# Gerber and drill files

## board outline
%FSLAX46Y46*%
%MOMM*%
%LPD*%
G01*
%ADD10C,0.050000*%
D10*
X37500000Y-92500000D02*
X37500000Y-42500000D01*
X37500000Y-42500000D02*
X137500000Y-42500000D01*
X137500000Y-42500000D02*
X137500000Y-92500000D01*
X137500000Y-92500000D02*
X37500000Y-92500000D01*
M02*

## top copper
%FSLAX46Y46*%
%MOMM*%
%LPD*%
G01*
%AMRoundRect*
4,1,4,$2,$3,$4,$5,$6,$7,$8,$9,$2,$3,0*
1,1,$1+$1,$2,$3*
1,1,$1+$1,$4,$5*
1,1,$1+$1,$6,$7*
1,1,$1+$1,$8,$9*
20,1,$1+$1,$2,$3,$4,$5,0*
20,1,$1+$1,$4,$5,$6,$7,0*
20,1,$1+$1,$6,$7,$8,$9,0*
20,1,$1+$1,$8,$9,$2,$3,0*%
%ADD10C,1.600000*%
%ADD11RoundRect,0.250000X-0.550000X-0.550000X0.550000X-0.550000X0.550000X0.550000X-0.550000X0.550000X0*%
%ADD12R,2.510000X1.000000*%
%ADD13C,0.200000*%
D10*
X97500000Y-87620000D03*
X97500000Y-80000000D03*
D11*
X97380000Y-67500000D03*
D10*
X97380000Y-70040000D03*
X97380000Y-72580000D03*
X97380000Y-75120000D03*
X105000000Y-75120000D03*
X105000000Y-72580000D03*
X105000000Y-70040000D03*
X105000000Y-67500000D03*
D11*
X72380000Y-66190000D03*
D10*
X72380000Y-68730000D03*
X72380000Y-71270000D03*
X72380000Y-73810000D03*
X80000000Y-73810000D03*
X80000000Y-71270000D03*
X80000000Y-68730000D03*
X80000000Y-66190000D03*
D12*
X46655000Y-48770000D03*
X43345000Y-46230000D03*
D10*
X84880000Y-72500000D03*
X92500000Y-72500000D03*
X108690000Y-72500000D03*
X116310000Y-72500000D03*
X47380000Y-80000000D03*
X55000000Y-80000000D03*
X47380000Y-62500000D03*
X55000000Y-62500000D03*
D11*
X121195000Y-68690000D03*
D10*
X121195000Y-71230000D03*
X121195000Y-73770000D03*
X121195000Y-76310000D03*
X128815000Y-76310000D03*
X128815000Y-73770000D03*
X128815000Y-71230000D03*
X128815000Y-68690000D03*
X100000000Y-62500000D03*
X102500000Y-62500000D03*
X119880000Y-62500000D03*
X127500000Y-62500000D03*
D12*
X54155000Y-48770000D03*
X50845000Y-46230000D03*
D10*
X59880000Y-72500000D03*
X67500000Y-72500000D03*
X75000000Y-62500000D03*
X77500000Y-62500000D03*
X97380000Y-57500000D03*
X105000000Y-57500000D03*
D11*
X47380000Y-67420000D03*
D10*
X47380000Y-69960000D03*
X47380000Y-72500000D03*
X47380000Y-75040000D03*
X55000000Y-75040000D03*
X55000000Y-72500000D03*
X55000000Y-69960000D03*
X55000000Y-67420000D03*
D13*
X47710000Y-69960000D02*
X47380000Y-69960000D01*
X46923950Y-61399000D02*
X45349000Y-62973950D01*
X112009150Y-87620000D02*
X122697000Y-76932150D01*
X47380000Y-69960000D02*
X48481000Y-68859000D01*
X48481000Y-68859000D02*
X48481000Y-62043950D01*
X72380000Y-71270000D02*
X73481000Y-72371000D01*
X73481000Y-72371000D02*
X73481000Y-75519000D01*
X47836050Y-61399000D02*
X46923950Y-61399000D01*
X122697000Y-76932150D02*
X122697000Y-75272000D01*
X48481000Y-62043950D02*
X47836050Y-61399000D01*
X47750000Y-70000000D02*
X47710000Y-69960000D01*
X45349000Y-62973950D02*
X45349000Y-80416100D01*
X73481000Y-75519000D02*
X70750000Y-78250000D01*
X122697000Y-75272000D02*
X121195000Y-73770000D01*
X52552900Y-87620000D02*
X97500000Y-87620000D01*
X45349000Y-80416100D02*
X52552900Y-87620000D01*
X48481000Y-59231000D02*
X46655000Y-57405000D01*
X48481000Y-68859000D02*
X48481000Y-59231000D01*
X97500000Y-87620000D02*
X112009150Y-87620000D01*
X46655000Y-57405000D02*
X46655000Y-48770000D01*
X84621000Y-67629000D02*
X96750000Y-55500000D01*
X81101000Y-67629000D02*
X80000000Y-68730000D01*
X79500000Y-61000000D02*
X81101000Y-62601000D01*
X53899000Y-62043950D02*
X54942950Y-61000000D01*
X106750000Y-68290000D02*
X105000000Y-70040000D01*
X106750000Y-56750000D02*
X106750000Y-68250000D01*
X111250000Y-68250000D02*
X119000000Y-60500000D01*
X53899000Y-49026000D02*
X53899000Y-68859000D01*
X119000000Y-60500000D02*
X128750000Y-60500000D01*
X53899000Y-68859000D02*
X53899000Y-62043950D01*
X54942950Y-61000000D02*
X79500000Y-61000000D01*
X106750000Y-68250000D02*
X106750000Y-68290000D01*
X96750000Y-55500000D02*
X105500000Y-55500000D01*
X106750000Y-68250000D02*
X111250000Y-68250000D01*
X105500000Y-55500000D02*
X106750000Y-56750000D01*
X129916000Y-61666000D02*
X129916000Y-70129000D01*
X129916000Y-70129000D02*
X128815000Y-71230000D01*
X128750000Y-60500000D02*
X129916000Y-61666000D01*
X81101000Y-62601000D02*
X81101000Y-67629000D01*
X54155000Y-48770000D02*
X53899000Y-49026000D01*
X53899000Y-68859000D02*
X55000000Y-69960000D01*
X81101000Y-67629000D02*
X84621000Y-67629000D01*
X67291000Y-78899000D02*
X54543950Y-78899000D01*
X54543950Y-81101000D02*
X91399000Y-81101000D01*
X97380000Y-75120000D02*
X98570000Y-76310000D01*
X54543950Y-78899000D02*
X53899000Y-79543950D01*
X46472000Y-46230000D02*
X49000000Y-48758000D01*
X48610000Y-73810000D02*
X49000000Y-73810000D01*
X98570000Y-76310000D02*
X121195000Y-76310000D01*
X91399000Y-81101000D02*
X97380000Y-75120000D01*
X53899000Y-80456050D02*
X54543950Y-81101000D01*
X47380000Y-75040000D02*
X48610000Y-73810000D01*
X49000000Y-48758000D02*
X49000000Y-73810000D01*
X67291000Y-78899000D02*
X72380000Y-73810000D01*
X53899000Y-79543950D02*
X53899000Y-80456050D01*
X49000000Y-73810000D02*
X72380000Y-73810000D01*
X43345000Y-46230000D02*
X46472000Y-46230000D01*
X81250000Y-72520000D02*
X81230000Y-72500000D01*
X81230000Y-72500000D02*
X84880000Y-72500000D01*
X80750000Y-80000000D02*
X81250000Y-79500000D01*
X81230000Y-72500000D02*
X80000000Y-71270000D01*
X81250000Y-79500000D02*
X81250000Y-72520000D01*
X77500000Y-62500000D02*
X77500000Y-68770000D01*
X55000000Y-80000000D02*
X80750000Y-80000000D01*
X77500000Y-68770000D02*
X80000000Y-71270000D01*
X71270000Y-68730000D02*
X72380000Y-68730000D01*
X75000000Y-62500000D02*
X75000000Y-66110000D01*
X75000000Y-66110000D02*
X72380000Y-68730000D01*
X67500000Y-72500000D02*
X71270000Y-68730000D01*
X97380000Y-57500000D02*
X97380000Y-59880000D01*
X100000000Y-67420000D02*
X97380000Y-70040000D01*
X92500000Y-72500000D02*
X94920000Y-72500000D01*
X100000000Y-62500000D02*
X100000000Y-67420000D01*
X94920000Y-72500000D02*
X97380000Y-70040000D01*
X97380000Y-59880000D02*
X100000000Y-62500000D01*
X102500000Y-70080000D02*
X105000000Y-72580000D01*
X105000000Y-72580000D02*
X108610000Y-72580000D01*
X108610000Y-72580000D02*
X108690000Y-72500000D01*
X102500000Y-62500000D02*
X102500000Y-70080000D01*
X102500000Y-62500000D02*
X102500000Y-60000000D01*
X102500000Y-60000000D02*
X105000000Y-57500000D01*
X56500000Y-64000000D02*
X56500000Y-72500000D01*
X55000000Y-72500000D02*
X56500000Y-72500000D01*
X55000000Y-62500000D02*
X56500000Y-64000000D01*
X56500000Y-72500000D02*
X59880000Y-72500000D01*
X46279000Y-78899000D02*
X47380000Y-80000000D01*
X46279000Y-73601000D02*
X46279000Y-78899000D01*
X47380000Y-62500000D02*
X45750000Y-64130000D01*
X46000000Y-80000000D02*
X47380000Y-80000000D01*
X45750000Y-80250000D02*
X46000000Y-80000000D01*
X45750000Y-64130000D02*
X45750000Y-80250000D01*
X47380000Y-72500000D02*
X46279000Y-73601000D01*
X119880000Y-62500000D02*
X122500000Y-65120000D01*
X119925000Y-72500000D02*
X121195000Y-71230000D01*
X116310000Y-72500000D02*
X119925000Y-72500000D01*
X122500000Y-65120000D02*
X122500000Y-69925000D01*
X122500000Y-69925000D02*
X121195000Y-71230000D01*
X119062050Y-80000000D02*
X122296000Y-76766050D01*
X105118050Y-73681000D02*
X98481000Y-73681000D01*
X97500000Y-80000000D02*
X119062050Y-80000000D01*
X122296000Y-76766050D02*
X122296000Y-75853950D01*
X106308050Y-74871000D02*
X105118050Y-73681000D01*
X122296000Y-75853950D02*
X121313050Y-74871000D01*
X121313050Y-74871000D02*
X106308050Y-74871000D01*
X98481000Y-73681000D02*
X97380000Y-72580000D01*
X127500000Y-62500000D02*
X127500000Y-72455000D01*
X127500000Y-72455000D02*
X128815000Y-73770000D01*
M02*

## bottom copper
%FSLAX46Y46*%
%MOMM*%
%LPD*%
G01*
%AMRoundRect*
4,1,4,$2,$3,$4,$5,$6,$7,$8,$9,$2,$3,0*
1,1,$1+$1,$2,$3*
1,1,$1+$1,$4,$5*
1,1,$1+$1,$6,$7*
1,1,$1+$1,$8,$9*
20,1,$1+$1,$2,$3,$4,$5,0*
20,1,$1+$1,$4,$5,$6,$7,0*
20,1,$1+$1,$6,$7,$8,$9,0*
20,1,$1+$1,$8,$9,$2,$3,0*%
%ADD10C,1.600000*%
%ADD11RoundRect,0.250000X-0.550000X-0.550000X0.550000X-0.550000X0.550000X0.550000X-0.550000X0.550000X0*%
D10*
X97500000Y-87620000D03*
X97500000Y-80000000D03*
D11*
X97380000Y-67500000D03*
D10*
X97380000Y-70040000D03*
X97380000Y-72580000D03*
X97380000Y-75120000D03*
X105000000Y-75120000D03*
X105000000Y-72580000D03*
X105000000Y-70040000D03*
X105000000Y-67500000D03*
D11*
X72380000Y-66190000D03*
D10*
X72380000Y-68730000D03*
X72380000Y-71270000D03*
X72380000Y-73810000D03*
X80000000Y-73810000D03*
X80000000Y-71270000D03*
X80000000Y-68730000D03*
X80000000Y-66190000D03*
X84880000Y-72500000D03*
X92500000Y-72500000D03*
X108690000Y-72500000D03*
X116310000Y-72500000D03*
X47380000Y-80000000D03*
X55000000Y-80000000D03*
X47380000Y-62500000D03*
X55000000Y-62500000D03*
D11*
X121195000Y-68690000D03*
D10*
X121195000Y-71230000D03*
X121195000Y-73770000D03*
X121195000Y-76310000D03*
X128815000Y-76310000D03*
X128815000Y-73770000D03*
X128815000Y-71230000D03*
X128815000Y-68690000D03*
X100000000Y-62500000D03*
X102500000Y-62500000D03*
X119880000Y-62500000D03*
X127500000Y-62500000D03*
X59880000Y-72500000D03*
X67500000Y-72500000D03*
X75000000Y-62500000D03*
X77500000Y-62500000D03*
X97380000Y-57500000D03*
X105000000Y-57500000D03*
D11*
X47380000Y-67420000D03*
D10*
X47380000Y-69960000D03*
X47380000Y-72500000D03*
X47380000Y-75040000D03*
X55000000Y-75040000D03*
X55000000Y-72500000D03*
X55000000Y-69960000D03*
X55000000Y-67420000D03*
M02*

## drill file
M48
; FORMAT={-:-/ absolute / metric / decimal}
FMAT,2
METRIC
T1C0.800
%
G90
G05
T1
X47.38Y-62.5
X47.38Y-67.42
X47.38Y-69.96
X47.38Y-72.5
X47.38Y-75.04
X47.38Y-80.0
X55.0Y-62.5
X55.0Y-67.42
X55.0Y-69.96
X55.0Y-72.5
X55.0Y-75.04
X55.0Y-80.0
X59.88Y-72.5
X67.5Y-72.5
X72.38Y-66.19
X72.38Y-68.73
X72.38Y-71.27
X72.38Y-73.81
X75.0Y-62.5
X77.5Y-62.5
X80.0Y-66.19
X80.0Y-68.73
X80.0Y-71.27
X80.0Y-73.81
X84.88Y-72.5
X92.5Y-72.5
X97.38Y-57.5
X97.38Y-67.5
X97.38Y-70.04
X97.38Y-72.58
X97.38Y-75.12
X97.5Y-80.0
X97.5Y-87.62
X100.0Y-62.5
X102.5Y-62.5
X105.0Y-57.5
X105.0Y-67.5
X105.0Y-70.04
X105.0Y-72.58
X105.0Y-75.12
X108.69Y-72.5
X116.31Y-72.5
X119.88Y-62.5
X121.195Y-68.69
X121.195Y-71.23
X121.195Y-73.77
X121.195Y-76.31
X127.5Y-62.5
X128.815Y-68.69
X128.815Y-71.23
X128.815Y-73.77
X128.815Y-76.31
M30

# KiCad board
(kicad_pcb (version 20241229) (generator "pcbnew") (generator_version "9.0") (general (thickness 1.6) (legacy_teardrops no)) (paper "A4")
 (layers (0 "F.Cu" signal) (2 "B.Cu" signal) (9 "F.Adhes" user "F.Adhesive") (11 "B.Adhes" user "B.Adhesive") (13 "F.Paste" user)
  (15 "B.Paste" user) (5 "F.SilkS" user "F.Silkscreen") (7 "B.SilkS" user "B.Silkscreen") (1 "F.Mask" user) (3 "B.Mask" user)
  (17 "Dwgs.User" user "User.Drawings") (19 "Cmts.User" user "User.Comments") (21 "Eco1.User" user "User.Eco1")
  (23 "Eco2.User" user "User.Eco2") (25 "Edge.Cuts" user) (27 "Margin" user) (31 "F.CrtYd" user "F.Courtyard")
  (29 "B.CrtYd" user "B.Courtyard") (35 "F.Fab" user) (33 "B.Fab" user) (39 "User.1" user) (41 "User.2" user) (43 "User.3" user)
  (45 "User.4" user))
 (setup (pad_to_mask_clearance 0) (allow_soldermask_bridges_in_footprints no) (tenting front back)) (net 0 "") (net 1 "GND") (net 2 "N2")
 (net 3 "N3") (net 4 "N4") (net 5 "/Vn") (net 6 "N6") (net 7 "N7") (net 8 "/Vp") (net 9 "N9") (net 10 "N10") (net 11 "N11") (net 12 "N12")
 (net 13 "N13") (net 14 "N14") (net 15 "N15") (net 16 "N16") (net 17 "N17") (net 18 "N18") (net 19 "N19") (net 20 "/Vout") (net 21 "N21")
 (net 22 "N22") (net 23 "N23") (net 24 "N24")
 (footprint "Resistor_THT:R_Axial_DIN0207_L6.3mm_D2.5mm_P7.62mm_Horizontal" (layer "F.Cu") (at 97.5 87.62 90)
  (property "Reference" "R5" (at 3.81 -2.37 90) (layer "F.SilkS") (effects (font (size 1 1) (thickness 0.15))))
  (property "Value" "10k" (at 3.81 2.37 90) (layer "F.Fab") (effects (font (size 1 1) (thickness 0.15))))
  (pad "1" thru_hole circle (at 0 0 90) (size 1.6 1.6) (drill 0.8) (layers "*.Cu" "*.Mask") (remove_unused_layers no) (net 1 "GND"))
  (pad "2" thru_hole circle (at 7.62 0 90) (size 1.6 1.6) (drill 0.8) (layers "*.Cu" "*.Mask") (remove_unused_layers no) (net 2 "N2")))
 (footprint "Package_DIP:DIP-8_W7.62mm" (layer "F.Cu") (at 97.38 67.5)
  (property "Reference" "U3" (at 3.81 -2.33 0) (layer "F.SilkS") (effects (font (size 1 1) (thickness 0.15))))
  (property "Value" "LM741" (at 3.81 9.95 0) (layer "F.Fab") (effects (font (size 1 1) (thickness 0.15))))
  (pad "1" thru_hole roundrect (at 0 0) (size 1.6 1.6) (drill 0.8) (layers "*.Cu" "*.Mask") (remove_unused_layers no)
   (roundrect_rratio 0.15625) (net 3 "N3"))
  (pad "2" thru_hole circle (at 0 2.54) (size 1.6 1.6) (drill 0.8) (layers "*.Cu" "*.Mask") (remove_unused_layers no) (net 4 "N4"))
  (pad "3" thru_hole circle (at 0 5.08) (size 1.6 1.6) (drill 0.8) (layers "*.Cu" "*.Mask") (remove_unused_layers no) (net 2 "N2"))
  (pad "4" thru_hole circle (at 0 7.62) (size 1.6 1.6) (drill 0.8) (layers "*.Cu" "*.Mask") (remove_unused_layers no) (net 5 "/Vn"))
  (pad "5" thru_hole circle (at 7.62 7.62) (size 1.6 1.6) (drill 0.8) (layers "*.Cu" "*.Mask") (remove_unused_layers no) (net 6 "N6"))
  (pad "6" thru_hole circle (at 7.62 5.08) (size 1.6 1.6) (drill 0.8) (layers "*.Cu" "*.Mask") (remove_unused_layers no) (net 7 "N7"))
  (pad "7" thru_hole circle (at 7.62 2.54) (size 1.6 1.6) (drill 0.8) (layers "*.Cu" "*.Mask") (remove_unused_layers no) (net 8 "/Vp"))
  (pad "8" thru_hole circle (at 7.62 0) (size 1.6 1.6) (drill 0.8) (layers "*.Cu" "*.Mask") (remove_unused_layers no) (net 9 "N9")))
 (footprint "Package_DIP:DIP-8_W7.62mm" (layer "F.Cu") (at 72.38 66.19)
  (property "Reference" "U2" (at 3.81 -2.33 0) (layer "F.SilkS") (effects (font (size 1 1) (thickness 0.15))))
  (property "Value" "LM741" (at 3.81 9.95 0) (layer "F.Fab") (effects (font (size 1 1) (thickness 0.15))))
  (pad "1" thru_hole roundrect (at 0 0) (size 1.6 1.6) (drill 0.8) (layers "*.Cu" "*.Mask") (remove_unused_layers no)
   (roundrect_rratio 0.15625) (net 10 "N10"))
  (pad "2" thru_hole circle (at 0 2.54) (size 1.6 1.6) (drill 0.8) (layers "*.Cu" "*.Mask") (remove_unused_layers no) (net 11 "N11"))
  (pad "3" thru_hole circle (at 0 5.08) (size 1.6 1.6) (drill 0.8) (layers "*.Cu" "*.Mask") (remove_unused_layers no) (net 1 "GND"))
  (pad "4" thru_hole circle (at 0 7.62) (size 1.6 1.6) (drill 0.8) (layers "*.Cu" "*.Mask") (remove_unused_layers no) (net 5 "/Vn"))
  (pad "5" thru_hole circle (at 7.62 7.62) (size 1.6 1.6) (drill 0.8) (layers "*.Cu" "*.Mask") (remove_unused_layers no) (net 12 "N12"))
  (pad "6" thru_hole circle (at 7.62 5.08) (size 1.6 1.6) (drill 0.8) (layers "*.Cu" "*.Mask") (remove_unused_layers no) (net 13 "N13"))
  (pad "7" thru_hole circle (at 7.62 2.54) (size 1.6 1.6) (drill 0.8) (layers "*.Cu" "*.Mask") (remove_unused_layers no) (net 8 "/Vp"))
  (pad "8" thru_hole circle (at 7.62 0) (size 1.6 1.6) (drill 0.8) (layers "*.Cu" "*.Mask") (remove_unused_layers no) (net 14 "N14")))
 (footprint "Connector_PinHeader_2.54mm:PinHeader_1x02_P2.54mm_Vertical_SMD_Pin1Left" (layer "F.Cu") (at 45 47.5 180)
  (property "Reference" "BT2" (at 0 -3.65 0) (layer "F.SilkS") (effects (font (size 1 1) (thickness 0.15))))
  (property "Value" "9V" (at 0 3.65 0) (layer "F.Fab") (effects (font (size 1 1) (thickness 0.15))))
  (pad "1" smd rect (at -1.655 -1.27 180) (size 2.51 1) (layers "F.Cu" "F.Mask" "F.Paste") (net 1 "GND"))
  (pad "2" smd rect (at 1.655 1.27 180) (size 2.51 1) (layers "F.Cu" "F.Mask" "F.Paste") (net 5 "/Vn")))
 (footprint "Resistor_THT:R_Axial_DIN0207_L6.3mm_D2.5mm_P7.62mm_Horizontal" (layer "F.Cu") (at 84.88 72.5)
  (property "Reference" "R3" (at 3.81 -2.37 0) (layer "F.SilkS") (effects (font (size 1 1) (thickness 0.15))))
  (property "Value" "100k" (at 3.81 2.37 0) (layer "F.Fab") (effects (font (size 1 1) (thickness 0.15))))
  (pad "1" thru_hole circle (at 0 0) (size 1.6 1.6) (drill 0.8) (layers "*.Cu" "*.Mask") (remove_unused_layers no) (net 13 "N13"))
  (pad "2" thru_hole circle (at 7.62 0) (size 1.6 1.6) (drill 0.8) (layers "*.Cu" "*.Mask") (remove_unused_layers no) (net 4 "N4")))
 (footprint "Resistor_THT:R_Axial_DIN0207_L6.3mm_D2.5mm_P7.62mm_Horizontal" (layer "F.Cu") (at 108.69 72.5)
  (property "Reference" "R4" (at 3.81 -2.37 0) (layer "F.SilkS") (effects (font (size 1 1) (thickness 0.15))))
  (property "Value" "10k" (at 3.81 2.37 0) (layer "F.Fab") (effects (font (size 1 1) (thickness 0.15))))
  (pad "1" thru_hole circle (at 0 0) (size 1.6 1.6) (drill 0.8) (layers "*.Cu" "*.Mask") (remove_unused_layers no) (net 7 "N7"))
  (pad "2" thru_hole circle (at 7.62 0) (size 1.6 1.6) (drill 0.8) (layers "*.Cu" "*.Mask") (remove_unused_layers no) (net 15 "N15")))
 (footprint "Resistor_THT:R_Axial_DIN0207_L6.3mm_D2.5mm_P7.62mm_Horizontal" (layer "F.Cu") (at 47.38 80)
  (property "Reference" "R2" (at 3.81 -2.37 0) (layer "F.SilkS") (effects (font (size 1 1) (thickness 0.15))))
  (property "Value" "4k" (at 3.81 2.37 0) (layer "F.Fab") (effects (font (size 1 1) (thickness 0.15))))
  (pad "1" thru_hole circle (at 0 0) (size 1.6 1.6) (drill 0.8) (layers "*.Cu" "*.Mask") (remove_unused_layers no) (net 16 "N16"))
  (pad "2" thru_hole circle (at 7.62 0) (size 1.6 1.6) (drill 0.8) (layers "*.Cu" "*.Mask") (remove_unused_layers no) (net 13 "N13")))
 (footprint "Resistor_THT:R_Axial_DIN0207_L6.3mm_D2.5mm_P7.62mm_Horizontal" (layer "F.Cu") (at 47.38 62.5)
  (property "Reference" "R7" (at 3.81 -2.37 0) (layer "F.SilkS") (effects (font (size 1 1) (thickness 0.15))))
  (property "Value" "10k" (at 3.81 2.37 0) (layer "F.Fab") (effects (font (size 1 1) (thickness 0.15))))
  (pad "1" thru_hole circle (at 0 0) (size 1.6 1.6) (drill 0.8) (layers "*.Cu" "*.Mask") (remove_unused_layers no) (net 16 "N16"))
  (pad "2" thru_hole circle (at 7.62 0) (size 1.6 1.6) (drill 0.8) (layers "*.Cu" "*.Mask") (remove_unused_layers no) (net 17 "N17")))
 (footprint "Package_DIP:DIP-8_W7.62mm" (layer "F.Cu") (at 121.195 68.69)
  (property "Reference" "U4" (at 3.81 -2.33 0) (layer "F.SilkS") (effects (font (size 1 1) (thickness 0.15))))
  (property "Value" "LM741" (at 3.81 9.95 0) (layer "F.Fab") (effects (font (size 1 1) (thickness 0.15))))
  (pad "1" thru_hole roundrect (at 0 0) (size 1.6 1.6) (drill 0.8) (layers "*.Cu" "*.Mask") (remove_unused_layers no)
   (roundrect_rratio 0.15625) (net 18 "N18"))
  (pad "2" thru_hole circle (at 0 2.54) (size 1.6 1.6) (drill 0.8) (layers "*.Cu" "*.Mask") (remove_unused_layers no) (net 15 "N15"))
  (pad "3" thru_hole circle (at 0 5.08) (size 1.6 1.6) (drill 0.8) (layers "*.Cu" "*.Mask") (remove_unused_layers no) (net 1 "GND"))
  (pad "4" thru_hole circle (at 0 7.62) (size 1.6 1.6) (drill 0.8) (layers "*.Cu" "*.Mask") (remove_unused_layers no) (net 5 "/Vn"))
  (pad "5" thru_hole circle (at 7.62 7.62) (size 1.6 1.6) (drill 0.8) (layers "*.Cu" "*.Mask") (remove_unused_layers no) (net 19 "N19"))
  (pad "6" thru_hole circle (at 7.62 5.08) (size 1.6 1.6) (drill 0.8) (layers "*.Cu" "*.Mask") (remove_unused_layers no) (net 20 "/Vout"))
  (pad "7" thru_hole circle (at 7.62 2.54) (size 1.6 1.6) (drill 0.8) (layers "*.Cu" "*.Mask") (remove_unused_layers no) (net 8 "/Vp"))
  (pad "8" thru_hole circle (at 7.62 0) (size 1.6 1.6) (drill 0.8) (layers "*.Cu" "*.Mask") (remove_unused_layers no) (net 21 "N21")))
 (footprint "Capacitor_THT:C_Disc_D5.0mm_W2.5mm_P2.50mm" (layer "F.Cu") (at 100 62.5)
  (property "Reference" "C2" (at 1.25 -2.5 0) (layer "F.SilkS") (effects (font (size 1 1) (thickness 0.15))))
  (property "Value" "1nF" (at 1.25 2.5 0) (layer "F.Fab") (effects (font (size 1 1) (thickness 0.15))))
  (pad "1" thru_hole circle (at 0 0) (size 1.6 1.6) (drill 0.8) (layers "*.Cu" "*.Mask") (remove_unused_layers no) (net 4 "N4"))
  (pad "2" thru_hole circle (at 2.5 0) (size 1.6 1.6) (drill 0.8) (layers "*.Cu" "*.Mask") (remove_unused_layers no) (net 7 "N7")))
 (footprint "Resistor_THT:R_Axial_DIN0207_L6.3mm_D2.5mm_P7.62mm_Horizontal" (layer "F.Cu") (at 119.88 62.5)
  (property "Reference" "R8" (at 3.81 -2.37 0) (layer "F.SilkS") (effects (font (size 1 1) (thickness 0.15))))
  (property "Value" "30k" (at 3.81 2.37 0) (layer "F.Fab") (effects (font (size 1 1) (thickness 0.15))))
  (pad "1" thru_hole circle (at 0 0) (size 1.6 1.6) (drill 0.8) (layers "*.Cu" "*.Mask") (remove_unused_layers no) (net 15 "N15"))
  (pad "2" thru_hole circle (at 7.62 0) (size 1.6 1.6) (drill 0.8) (layers "*.Cu" "*.Mask") (remove_unused_layers no) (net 20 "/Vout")))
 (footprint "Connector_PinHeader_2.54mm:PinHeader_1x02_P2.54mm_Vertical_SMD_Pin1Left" (layer "F.Cu") (at 52.5 47.5 180)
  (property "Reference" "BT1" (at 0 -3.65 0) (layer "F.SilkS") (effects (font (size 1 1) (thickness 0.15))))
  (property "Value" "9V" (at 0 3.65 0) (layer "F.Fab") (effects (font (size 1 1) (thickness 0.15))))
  (pad "1" smd rect (at -1.655 -1.27 180) (size 2.51 1) (layers "F.Cu" "F.Mask" "F.Paste") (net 8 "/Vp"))
  (pad "2" smd rect (at 1.655 1.27 180) (size 2.51 1) (layers "F.Cu" "F.Mask" "F.Paste") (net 1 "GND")))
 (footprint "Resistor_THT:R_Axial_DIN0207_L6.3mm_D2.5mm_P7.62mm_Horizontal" (layer "F.Cu") (at 59.88 72.5)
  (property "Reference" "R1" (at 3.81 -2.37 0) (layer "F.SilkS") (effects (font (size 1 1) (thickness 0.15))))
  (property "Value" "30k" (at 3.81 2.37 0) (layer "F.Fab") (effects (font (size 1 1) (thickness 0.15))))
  (pad "1" thru_hole circle (at 0 0) (size 1.6 1.6) (drill 0.8) (layers "*.Cu" "*.Mask") (remove_unused_layers no) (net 17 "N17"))
  (pad "2" thru_hole circle (at 7.62 0) (size 1.6 1.6) (drill 0.8) (layers "*.Cu" "*.Mask") (remove_unused_layers no) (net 11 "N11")))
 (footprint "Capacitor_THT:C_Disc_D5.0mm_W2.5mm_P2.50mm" (layer "F.Cu") (at 75 62.5)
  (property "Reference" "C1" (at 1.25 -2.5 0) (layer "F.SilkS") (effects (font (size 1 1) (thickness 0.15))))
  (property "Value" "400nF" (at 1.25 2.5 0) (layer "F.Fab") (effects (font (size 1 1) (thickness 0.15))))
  (pad "1" thru_hole circle (at 0 0) (size 1.6 1.6) (drill 0.8) (layers "*.Cu" "*.Mask") (remove_unused_layers no) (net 11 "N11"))
  (pad "2" thru_hole circle (at 2.5 0) (size 1.6 1.6) (drill 0.8) (layers "*.Cu" "*.Mask") (remove_unused_layers no) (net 13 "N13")))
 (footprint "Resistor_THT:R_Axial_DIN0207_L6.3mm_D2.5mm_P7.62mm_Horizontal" (layer "F.Cu") (at 97.38 57.5)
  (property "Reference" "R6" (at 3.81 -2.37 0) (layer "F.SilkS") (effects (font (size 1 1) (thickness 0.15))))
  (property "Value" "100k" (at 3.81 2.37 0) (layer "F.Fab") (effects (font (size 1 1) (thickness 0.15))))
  (pad "1" thru_hole circle (at 0 0) (size 1.6 1.6) (drill 0.8) (layers "*.Cu" "*.Mask") (remove_unused_layers no) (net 4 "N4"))
  (pad "2" thru_hole circle (at 7.62 0) (size 1.6 1.6) (drill 0.8) (layers "*.Cu" "*.Mask") (remove_unused_layers no) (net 7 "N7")))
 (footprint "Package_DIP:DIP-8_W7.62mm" (layer "F.Cu") (at 47.38 67.42)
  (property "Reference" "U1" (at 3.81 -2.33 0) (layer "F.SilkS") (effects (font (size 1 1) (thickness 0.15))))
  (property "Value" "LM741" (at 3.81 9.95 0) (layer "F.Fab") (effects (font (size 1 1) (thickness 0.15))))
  (pad "1" thru_hole roundrect (at 0 0) (size 1.6 1.6) (drill 0.8) (layers "*.Cu" "*.Mask") (remove_unused_layers no)
   (roundrect_rratio 0.15625) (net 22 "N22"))
  (pad "2" thru_hole circle (at 0 2.54) (size 1.6 1.6) (drill 0.8) (layers "*.Cu" "*.Mask") (remove_unused_layers no) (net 1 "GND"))
  (pad "3" thru_hole circle (at 0 5.08) (size 1.6 1.6) (drill 0.8) (layers "*.Cu" "*.Mask") (remove_unused_layers no) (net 16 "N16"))
  (pad "4" thru_hole circle (at 0 7.62) (size 1.6 1.6) (drill 0.8) (layers "*.Cu" "*.Mask") (remove_unused_layers no) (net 5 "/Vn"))
  (pad "5" thru_hole circle (at 7.62 7.62) (size 1.6 1.6) (drill 0.8) (layers "*.Cu" "*.Mask") (remove_unused_layers no) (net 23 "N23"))
  (pad "6" thru_hole circle (at 7.62 5.08) (size 1.6 1.6) (drill 0.8) (layers "*.Cu" "*.Mask") (remove_unused_layers no) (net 17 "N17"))
  (pad "7" thru_hole circle (at 7.62 2.54) (size 1.6 1.6) (drill 0.8) (layers "*.Cu" "*.Mask") (remove_unused_layers no) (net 8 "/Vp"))
  (pad "8" thru_hole circle (at 7.62 0) (size 1.6 1.6) (drill 0.8) (layers "*.Cu" "*.Mask") (remove_unused_layers no) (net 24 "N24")))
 (gr_line (start 37.5 92.5) (end 37.5 42.5) (stroke (width 0.05) (type default)) (layer "Edge.Cuts"))
 (gr_line (start 37.5 42.5) (end 137.5 42.5) (stroke (width 0.05) (type default)) (layer "Edge.Cuts"))
 (gr_line (start 137.5 42.5) (end 137.5 92.5) (stroke (width 0.05) (type default)) (layer "Edge.Cuts"))
 (gr_line (start 137.5 92.5) (end 37.5 92.5) (stroke (width 0.05) (type default)) (layer "Edge.Cuts"))
 (segment (start 47.71 69.96) (end 47.38 69.96) (width 0.2) (layer "F.Cu") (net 1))
 (segment (start 46.92395 61.399) (end 45.349 62.97395) (width 0.2) (layer "F.Cu") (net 1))
 (segment (start 112.00915 87.62) (end 122.697 76.93215) (width 0.2) (layer "F.Cu") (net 1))
 (segment (start 47.38 69.96) (end 48.481 68.859) (width 0.2) (layer "F.Cu") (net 1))
 (segment (start 48.481 68.859) (end 48.481 62.04395) (width 0.2) (layer "F.Cu") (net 1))
 (segment (start 72.38 71.27) (end 73.481 72.371) (width 0.2) (layer "F.Cu") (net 1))
 (segment (start 73.481 72.371) (end 73.481 75.519) (width 0.2) (layer "F.Cu") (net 1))
 (segment (start 47.83605 61.399) (end 46.92395 61.399) (width 0.2) (layer "F.Cu") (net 1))
 (segment (start 122.697 76.93215) (end 122.697 75.272) (width 0.2) (layer "F.Cu") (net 1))
 (segment (start 48.481 62.04395) (end 47.83605 61.399) (width 0.2) (layer "F.Cu") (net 1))
 (segment (start 47.75 70) (end 47.71 69.96) (width 0.2) (layer "F.Cu") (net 1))
 (segment (start 45.349 62.97395) (end 45.349 80.4161) (width 0.2) (layer "F.Cu") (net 1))
 (segment (start 73.481 75.519) (end 70.75 78.25) (width 0.2) (layer "F.Cu") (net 1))
 (segment (start 122.697 75.272) (end 121.195 73.77) (width 0.2) (layer "F.Cu") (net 1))
 (segment (start 52.5529 87.62) (end 97.5 87.62) (width 0.2) (layer "F.Cu") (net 1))
 (segment (start 45.349 80.4161) (end 52.5529 87.62) (width 0.2) (layer "F.Cu") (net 1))
 (segment (start 48.481 59.231) (end 46.655 57.405) (width 0.2) (layer "F.Cu") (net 1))
 (segment (start 48.481 68.859) (end 48.481 59.231) (width 0.2) (layer "F.Cu") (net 1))
 (segment (start 97.5 87.62) (end 112.00915 87.62) (width 0.2) (layer "F.Cu") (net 1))
 (segment (start 46.655 57.405) (end 46.655 48.77) (width 0.2) (layer "F.Cu") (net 1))
 (segment (start 84.621 67.629) (end 96.75 55.5) (width 0.2) (layer "F.Cu") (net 8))
 (segment (start 81.101 67.629) (end 80 68.73) (width 0.2) (layer "F.Cu") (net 8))
 (segment (start 79.5 61) (end 81.101 62.601) (width 0.2) (layer "F.Cu") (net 8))
 (segment (start 53.899 62.04395) (end 54.94295 61) (width 0.2) (layer "F.Cu") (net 8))
 (segment (start 106.75 68.29) (end 105 70.04) (width 0.2) (layer "F.Cu") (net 8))
 (segment (start 106.75 56.75) (end 106.75 68.25) (width 0.2) (layer "F.Cu") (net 8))
 (segment (start 111.25 68.25) (end 119 60.5) (width 0.2) (layer "F.Cu") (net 8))
 (segment (start 53.899 49.026) (end 53.899 68.859) (width 0.2) (layer "F.Cu") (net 8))
 (segment (start 119 60.5) (end 128.75 60.5) (width 0.2) (layer "F.Cu") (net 8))
 (segment (start 53.899 68.859) (end 53.899 62.04395) (width 0.2) (layer "F.Cu") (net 8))
 (segment (start 54.94295 61) (end 79.5 61) (width 0.2) (layer "F.Cu") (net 8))
 (segment (start 106.75 68.25) (end 106.75 68.29) (width 0.2) (layer "F.Cu") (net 8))
 (segment (start 96.75 55.5) (end 105.5 55.5) (width 0.2) (layer "F.Cu") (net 8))
 (segment (start 106.75 68.25) (end 111.25 68.25) (width 0.2) (layer "F.Cu") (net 8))
 (segment (start 105.5 55.5) (end 106.75 56.75) (width 0.2) (layer "F.Cu") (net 8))
 (segment (start 129.916 61.666) (end 129.916 70.129) (width 0.2) (layer "F.Cu") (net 8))
 (segment (start 129.916 70.129) (end 128.815 71.23) (width 0.2) (layer "F.Cu") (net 8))
 (segment (start 128.75 60.5) (end 129.916 61.666) (width 0.2) (layer "F.Cu") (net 8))
 (segment (start 81.101 62.601) (end 81.101 67.629) (width 0.2) (layer "F.Cu") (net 8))
 (segment (start 54.155 48.77) (end 53.899 49.026) (width 0.2) (layer "F.Cu") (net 8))
 (segment (start 53.899 68.859) (end 55 69.96) (width 0.2) (layer "F.Cu") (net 8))
 (segment (start 81.101 67.629) (end 84.621 67.629) (width 0.2) (layer "F.Cu") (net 8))
 (segment (start 67.291 78.899) (end 54.54395 78.899) (width 0.2) (layer "F.Cu") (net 5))
 (segment (start 54.54395 81.101) (end 91.399 81.101) (width 0.2) (layer "F.Cu") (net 5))
 (segment (start 97.38 75.12) (end 98.57 76.31) (width 0.2) (layer "F.Cu") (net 5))
 (segment (start 54.54395 78.899) (end 53.899 79.54395) (width 0.2) (layer "F.Cu") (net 5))
 (segment (start 46.472 46.23) (end 49 48.758) (width 0.2) (layer "F.Cu") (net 5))
 (segment (start 48.61 73.81) (end 49 73.81) (width 0.2) (layer "F.Cu") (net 5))
 (segment (start 98.57 76.31) (end 121.195 76.31) (width 0.2) (layer "F.Cu") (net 5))
 (segment (start 91.399 81.101) (end 97.38 75.12) (width 0.2) (layer "F.Cu") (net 5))
 (segment (start 53.899 80.45605) (end 54.54395 81.101) (width 0.2) (layer "F.Cu") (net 5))
 (segment (start 47.38 75.04) (end 48.61 73.81) (width 0.2) (layer "F.Cu") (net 5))
 (segment (start 49 48.758) (end 49 73.81) (width 0.2) (layer "F.Cu") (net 5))
 (segment (start 67.291 78.899) (end 72.38 73.81) (width 0.2) (layer "F.Cu") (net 5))
 (segment (start 53.899 79.54395) (end 53.899 80.45605) (width 0.2) (layer "F.Cu") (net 5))
 (segment (start 49 73.81) (end 72.38 73.81) (width 0.2) (layer "F.Cu") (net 5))
 (segment (start 43.345 46.23) (end 46.472 46.23) (width 0.2) (layer "F.Cu") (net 5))
 (segment (start 81.25 72.52) (end 81.23 72.5) (width 0.2) (layer "F.Cu") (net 13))
 (segment (start 81.23 72.5) (end 84.88 72.5) (width 0.2) (layer "F.Cu") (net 13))
 (segment (start 80.75 80) (end 81.25 79.5) (width 0.2) (layer "F.Cu") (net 13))
 (segment (start 81.23 72.5) (end 80 71.27) (width 0.2) (layer "F.Cu") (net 13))
 (segment (start 81.25 79.5) (end 81.25 72.52) (width 0.2) (layer "F.Cu") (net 13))
 (segment (start 77.5 62.5) (end 77.5 68.77) (width 0.2) (layer "F.Cu") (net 13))
 (segment (start 55 80) (end 80.75 80) (width 0.2) (layer "F.Cu") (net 13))
 (segment (start 77.5 68.77) (end 80 71.27) (width 0.2) (layer "F.Cu") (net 13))
 (segment (start 71.27 68.73) (end 72.38 68.73) (width 0.2) (layer "F.Cu") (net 11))
 (segment (start 75 62.5) (end 75 66.11) (width 0.2) (layer "F.Cu") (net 11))
 (segment (start 75 66.11) (end 72.38 68.73) (width 0.2) (layer "F.Cu") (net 11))
 (segment (start 67.5 72.5) (end 71.27 68.73) (width 0.2) (layer "F.Cu") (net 11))
 (segment (start 97.38 57.5) (end 97.38 59.88) (width 0.2) (layer "F.Cu") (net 4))
 (segment (start 100 67.42) (end 97.38 70.04) (width 0.2) (layer "F.Cu") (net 4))
 (segment (start 92.5 72.5) (end 94.92 72.5) (width 0.2) (layer "F.Cu") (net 4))
 (segment (start 100 62.5) (end 100 67.42) (width 0.2) (layer "F.Cu") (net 4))
 (segment (start 94.92 72.5) (end 97.38 70.04) (width 0.2) (layer "F.Cu") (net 4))
 (segment (start 97.38 59.88) (end 100 62.5) (width 0.2) (layer "F.Cu") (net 4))
 (segment (start 102.5 70.08) (end 105 72.58) (width 0.2) (layer "F.Cu") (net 7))
 (segment (start 105 72.58) (end 108.61 72.58) (width 0.2) (layer "F.Cu") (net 7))
 (segment (start 108.61 72.58) (end 108.69 72.5) (width 0.2) (layer "F.Cu") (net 7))
 (segment (start 102.5 62.5) (end 102.5 70.08) (width 0.2) (layer "F.Cu") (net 7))
 (segment (start 102.5 62.5) (end 102.5 60) (width 0.2) (layer "F.Cu") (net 7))
 (segment (start 102.5 60) (end 105 57.5) (width 0.2) (layer "F.Cu") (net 7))
 (segment (start 56.5 64) (end 56.5 72.5) (width 0.2) (layer "F.Cu") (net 17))
 (segment (start 55 72.5) (end 56.5 72.5) (width 0.2) (layer "F.Cu") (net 17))
 (segment (start 55 62.5) (end 56.5 64) (width 0.2) (layer "F.Cu") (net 17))
 (segment (start 56.5 72.5) (end 59.88 72.5) (width 0.2) (layer "F.Cu") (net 17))
 (segment (start 46.279 78.899) (end 47.38 80) (width 0.2) (layer "F.Cu") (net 16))
 (segment (start 46.279 73.601) (end 46.279 78.899) (width 0.2) (layer "F.Cu") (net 16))
 (segment (start 47.38 62.5) (end 45.75 64.13) (width 0.2) (layer "F.Cu") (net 16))
 (segment (start 46 80) (end 47.38 80) (width 0.2) (layer "F.Cu") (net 16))
 (segment (start 45.75 80.25) (end 46 80) (width 0.2) (layer "F.Cu") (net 16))
 (segment (start 45.75 64.13) (end 45.75 80.25) (width 0.2) (layer "F.Cu") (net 16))
 (segment (start 47.38 72.5) (end 46.279 73.601) (width 0.2) (layer "F.Cu") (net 16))
 (segment (start 119.88 62.5) (end 122.5 65.12) (width 0.2) (layer "F.Cu") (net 15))
 (segment (start 119.925 72.5) (end 121.195 71.23) (width 0.2) (layer "F.Cu") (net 15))
 (segment (start 116.31 72.5) (end 119.925 72.5) (width 0.2) (layer "F.Cu") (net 15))
 (segment (start 122.5 65.12) (end 122.5 69.925) (width 0.2) (layer "F.Cu") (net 15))
 (segment (start 122.5 69.925) (end 121.195 71.23) (width 0.2) (layer "F.Cu") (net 15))
 (segment (start 119.06205 80) (end 122.296 76.76605) (width 0.2) (layer "F.Cu") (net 2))
 (segment (start 105.11805 73.681) (end 98.481 73.681) (width 0.2) (layer "F.Cu") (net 2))
 (segment (start 97.5 80) (end 119.06205 80) (width 0.2) (layer "F.Cu") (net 2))
 (segment (start 122.296 76.76605) (end 122.296 75.85395) (width 0.2) (layer "F.Cu") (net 2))
 (segment (start 106.30805 74.871) (end 105.11805 73.681) (width 0.2) (layer "F.Cu") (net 2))
 (segment (start 122.296 75.85395) (end 121.31305 74.871) (width 0.2) (layer "F.Cu") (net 2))
 (segment (start 121.31305 74.871) (end 106.30805 74.871) (width 0.2) (layer "F.Cu") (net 2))
 (segment (start 98.481 73.681) (end 97.38 72.58) (width 0.2) (layer "F.Cu") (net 2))
 (segment (start 127.5 62.5) (end 127.5 72.455) (width 0.2) (layer "F.Cu") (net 20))
 (segment (start 127.5 72.455) (end 128.815 73.77) (width 0.2) (layer "F.Cu") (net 20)))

